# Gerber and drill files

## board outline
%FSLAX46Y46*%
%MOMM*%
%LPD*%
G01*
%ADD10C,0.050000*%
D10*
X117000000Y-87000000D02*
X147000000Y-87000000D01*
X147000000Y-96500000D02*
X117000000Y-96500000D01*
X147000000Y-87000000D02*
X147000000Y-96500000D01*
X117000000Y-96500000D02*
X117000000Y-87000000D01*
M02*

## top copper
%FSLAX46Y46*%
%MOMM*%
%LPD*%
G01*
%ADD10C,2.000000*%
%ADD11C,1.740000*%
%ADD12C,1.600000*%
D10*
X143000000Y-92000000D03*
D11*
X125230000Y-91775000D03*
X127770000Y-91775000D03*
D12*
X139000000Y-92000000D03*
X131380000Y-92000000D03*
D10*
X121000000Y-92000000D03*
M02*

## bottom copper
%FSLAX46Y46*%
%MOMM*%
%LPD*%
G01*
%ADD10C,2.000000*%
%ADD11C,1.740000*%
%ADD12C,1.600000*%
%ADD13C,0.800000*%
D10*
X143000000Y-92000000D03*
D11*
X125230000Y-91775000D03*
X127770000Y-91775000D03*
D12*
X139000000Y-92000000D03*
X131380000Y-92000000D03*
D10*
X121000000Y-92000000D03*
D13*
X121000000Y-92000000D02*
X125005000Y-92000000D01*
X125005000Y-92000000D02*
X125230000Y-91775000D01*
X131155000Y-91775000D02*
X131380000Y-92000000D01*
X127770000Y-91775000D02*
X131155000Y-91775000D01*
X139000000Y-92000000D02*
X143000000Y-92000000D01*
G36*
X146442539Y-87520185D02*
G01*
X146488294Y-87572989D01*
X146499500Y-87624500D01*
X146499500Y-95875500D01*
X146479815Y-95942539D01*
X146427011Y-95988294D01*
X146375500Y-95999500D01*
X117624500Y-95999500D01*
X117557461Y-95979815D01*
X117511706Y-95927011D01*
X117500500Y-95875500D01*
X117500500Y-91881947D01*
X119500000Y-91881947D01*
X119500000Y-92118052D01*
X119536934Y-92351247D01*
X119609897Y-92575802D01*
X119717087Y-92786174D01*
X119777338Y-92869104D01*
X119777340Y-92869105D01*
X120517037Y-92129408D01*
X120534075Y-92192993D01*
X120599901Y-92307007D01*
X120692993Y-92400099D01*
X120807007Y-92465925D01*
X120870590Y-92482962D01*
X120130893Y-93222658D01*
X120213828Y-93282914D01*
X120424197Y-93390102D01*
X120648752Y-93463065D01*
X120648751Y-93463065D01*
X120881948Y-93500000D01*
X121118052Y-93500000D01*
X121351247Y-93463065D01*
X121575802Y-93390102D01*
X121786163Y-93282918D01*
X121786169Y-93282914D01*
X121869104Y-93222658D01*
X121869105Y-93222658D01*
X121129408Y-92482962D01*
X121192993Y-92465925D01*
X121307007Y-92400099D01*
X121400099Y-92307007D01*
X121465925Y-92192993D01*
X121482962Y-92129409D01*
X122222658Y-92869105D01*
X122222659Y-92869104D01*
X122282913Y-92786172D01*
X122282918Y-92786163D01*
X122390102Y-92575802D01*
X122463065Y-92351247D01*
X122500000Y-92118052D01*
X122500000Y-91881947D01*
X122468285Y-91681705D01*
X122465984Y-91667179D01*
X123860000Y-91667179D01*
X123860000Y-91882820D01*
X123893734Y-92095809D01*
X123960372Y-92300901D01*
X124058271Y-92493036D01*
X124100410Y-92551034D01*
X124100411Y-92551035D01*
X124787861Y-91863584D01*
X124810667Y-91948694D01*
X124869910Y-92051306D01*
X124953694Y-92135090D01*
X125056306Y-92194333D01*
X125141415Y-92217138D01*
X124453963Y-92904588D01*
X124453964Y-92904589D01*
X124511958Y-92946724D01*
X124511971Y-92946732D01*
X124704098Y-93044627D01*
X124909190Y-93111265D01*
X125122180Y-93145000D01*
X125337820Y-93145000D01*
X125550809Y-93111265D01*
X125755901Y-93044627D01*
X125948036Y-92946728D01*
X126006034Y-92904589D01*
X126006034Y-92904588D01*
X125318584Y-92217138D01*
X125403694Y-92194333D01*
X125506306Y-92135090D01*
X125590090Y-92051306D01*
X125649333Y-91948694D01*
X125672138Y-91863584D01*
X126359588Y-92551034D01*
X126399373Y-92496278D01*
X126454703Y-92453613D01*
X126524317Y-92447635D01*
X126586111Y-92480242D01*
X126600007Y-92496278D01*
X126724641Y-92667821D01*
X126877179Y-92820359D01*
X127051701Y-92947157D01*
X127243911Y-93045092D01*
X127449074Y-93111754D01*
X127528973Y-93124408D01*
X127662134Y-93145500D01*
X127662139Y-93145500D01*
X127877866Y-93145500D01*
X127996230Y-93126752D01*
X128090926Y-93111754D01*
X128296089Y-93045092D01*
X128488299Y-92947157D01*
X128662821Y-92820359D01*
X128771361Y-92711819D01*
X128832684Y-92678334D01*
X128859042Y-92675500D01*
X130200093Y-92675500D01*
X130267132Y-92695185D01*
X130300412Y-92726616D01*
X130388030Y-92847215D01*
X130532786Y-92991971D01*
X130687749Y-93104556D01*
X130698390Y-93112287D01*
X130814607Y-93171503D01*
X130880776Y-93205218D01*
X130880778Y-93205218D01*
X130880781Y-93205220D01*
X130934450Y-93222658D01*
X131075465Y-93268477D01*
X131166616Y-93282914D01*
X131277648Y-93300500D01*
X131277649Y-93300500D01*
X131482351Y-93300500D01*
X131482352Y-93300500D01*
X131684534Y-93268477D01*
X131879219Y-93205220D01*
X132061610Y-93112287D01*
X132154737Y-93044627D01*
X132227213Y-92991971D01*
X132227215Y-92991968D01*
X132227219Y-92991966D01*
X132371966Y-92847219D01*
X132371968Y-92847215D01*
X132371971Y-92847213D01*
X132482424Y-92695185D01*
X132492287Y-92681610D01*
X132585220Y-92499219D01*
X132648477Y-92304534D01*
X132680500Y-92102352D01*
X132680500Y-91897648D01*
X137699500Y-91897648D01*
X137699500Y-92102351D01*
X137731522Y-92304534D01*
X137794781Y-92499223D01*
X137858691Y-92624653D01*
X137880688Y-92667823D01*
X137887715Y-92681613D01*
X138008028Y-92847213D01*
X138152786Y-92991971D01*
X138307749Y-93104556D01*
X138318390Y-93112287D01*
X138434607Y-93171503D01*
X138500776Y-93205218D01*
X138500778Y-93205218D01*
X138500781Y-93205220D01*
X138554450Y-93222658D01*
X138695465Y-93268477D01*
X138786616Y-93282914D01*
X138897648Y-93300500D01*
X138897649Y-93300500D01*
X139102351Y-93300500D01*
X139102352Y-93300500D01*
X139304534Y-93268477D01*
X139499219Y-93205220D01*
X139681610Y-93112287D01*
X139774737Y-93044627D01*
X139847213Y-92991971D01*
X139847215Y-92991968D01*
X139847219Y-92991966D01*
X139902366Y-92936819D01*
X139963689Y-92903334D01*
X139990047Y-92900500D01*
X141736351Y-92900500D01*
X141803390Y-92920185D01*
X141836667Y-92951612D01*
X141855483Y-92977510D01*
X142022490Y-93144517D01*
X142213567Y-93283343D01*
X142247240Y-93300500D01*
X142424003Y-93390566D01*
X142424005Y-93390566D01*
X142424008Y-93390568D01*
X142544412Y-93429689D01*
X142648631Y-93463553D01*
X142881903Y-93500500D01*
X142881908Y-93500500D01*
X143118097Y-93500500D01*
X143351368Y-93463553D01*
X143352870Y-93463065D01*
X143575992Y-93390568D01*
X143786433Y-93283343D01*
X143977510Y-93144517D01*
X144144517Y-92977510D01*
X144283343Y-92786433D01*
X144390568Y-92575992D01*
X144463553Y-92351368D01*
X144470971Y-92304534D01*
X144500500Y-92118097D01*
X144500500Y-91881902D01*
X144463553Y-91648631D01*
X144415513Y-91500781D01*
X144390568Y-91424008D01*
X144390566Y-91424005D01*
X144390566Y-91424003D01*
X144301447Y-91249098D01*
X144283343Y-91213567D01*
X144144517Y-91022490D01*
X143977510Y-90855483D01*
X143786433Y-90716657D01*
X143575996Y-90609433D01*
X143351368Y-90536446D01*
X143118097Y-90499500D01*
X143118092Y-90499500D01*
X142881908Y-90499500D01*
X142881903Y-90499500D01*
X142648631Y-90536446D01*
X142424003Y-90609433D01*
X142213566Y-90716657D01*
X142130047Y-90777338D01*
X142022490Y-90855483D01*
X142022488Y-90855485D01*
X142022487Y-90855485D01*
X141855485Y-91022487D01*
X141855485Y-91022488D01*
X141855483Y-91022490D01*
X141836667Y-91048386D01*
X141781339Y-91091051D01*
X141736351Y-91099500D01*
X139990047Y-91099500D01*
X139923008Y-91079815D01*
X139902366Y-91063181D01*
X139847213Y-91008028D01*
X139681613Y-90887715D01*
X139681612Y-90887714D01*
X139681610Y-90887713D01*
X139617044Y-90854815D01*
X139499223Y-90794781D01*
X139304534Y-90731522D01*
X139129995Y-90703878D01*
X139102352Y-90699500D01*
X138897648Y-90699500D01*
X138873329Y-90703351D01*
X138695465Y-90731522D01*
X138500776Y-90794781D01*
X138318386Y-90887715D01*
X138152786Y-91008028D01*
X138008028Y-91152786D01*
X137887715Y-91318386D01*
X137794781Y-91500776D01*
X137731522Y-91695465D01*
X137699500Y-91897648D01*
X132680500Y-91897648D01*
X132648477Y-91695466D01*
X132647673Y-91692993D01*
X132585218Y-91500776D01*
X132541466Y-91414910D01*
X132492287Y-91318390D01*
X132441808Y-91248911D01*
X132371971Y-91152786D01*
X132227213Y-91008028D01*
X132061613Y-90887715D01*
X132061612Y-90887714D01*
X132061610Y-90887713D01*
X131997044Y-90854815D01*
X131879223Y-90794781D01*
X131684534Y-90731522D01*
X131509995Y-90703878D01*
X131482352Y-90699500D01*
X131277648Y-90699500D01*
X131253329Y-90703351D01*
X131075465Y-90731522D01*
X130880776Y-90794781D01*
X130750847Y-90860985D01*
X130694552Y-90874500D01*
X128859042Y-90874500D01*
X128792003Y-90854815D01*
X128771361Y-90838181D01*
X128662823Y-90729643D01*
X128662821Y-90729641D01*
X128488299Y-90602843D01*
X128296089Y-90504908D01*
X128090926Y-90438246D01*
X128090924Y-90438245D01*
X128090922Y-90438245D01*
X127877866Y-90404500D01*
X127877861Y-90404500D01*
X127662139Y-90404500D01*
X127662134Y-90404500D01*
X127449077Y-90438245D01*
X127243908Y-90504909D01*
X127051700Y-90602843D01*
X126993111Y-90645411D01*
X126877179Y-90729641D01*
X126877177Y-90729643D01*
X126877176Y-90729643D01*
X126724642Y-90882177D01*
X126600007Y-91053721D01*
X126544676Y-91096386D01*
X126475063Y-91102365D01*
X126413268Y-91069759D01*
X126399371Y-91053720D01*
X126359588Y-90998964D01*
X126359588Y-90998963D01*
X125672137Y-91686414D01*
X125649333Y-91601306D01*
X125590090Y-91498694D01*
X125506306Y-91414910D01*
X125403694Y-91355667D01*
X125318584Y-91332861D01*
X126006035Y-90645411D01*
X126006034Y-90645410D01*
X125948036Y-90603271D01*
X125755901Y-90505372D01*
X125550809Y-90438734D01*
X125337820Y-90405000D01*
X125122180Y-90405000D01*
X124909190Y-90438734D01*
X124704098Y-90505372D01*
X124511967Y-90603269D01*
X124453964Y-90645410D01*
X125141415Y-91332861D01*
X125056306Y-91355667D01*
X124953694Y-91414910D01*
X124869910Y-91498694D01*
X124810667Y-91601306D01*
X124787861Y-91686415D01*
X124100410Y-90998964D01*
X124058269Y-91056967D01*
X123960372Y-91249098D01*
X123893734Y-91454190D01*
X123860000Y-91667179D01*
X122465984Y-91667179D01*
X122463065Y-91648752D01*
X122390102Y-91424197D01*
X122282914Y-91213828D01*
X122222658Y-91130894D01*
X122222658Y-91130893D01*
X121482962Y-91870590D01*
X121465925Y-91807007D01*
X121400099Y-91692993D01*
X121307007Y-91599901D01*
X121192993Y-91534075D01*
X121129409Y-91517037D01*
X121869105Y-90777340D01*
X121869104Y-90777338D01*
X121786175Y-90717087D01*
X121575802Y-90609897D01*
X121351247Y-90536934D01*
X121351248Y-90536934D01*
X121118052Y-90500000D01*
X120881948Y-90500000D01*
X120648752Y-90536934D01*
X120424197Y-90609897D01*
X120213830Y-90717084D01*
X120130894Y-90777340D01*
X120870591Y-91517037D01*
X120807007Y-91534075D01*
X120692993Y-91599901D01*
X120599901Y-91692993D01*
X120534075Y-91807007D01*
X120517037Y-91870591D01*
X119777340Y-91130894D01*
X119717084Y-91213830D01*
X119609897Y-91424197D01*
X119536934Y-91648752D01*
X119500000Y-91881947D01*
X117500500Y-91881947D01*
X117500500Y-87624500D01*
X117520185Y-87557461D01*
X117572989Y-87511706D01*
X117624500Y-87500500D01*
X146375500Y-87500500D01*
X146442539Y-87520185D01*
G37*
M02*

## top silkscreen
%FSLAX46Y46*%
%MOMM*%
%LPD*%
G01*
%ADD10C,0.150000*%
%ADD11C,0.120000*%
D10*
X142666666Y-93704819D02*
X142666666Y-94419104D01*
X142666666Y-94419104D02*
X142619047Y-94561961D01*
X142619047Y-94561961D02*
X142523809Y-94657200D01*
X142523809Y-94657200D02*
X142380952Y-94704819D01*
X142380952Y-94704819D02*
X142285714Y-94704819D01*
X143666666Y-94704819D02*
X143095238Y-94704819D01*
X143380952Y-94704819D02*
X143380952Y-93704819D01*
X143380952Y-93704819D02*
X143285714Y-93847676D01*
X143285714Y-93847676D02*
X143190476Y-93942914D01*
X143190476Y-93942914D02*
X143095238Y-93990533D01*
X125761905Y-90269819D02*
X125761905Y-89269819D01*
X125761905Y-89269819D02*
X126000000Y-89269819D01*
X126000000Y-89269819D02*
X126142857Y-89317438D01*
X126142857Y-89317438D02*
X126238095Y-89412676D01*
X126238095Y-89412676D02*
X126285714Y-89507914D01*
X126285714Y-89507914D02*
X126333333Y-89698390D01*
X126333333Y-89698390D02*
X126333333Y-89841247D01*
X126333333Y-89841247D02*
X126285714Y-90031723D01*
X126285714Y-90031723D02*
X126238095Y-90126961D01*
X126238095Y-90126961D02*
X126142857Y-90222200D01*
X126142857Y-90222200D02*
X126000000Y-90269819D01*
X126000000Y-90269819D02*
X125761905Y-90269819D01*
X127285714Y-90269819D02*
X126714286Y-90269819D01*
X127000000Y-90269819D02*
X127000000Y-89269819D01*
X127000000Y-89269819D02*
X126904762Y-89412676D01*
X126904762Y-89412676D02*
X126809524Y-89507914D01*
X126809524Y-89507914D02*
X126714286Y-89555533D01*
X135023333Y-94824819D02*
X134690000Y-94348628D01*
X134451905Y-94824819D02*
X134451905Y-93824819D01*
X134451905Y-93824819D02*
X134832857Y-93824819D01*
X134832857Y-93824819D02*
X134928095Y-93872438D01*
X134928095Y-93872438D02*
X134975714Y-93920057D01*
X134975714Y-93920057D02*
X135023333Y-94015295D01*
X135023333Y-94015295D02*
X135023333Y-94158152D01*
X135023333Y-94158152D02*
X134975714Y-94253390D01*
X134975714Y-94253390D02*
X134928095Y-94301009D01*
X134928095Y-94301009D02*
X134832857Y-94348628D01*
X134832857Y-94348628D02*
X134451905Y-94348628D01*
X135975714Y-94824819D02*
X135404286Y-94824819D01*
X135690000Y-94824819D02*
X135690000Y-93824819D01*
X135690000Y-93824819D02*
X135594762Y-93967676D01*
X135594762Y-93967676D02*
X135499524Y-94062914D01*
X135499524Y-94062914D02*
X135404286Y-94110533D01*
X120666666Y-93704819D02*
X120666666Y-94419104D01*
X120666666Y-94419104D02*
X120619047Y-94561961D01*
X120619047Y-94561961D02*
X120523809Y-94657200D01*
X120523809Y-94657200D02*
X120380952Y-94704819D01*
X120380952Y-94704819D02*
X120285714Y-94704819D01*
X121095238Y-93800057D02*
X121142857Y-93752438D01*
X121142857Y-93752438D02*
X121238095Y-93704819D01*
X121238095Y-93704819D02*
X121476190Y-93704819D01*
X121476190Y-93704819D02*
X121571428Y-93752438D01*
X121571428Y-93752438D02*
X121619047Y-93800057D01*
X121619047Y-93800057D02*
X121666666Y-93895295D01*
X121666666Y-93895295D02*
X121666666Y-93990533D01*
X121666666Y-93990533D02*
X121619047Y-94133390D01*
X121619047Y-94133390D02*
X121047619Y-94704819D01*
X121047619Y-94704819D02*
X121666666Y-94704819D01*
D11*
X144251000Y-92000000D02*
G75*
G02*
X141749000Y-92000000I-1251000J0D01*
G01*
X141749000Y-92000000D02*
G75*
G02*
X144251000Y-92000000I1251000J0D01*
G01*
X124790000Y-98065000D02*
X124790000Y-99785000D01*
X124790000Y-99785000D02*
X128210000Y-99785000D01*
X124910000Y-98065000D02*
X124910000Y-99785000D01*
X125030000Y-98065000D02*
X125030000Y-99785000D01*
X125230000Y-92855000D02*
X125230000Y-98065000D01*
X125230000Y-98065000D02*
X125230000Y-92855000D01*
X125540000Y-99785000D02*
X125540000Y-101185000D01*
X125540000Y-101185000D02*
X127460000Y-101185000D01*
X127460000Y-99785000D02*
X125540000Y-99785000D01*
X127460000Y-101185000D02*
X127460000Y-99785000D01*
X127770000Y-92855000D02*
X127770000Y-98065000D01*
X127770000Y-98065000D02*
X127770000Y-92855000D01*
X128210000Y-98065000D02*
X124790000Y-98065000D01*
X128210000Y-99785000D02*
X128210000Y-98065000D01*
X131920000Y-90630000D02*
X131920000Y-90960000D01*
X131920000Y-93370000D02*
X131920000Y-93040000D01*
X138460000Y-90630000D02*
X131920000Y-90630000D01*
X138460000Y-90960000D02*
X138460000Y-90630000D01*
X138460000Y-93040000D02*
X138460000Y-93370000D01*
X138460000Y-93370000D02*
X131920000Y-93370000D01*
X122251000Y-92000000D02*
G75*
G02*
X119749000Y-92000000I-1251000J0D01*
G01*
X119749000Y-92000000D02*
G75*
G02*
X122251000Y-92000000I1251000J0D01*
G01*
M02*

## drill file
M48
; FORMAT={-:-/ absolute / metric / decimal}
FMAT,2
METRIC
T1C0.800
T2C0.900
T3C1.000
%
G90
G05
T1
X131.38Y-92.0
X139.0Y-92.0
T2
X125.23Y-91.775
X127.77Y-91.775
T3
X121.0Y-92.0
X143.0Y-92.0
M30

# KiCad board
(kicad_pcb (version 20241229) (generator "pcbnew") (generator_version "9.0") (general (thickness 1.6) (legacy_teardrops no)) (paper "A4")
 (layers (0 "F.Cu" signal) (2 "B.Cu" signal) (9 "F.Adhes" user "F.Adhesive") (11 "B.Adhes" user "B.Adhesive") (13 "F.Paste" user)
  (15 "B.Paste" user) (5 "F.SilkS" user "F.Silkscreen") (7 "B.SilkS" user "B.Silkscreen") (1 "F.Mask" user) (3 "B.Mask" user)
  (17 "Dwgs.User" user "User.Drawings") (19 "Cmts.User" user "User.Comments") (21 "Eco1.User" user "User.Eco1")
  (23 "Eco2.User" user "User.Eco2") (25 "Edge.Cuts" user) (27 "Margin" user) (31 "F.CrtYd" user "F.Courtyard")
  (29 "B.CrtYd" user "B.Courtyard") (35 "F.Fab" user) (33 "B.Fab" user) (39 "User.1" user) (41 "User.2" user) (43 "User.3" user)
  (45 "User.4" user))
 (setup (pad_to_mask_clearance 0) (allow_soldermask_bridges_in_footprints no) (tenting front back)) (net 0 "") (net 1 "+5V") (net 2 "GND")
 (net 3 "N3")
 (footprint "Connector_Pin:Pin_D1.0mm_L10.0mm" (layer "F.Cu") (at 143 92)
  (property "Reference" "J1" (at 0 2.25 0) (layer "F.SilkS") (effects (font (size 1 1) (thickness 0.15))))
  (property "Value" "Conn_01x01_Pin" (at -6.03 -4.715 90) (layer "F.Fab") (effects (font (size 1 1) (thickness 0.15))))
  (fp_circle (center 0 0) (end 1.25 0.05) (stroke (width 0.12) (type solid)) (fill no) (layer "F.SilkS"))
  (pad "1" thru_hole circle (at 0 0) (size 2 2) (drill 1) (layers "*.Cu" "*.Mask") (remove_unused_layers no) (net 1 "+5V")))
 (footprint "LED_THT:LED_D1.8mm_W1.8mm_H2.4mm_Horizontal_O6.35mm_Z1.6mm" (layer "F.Cu") (at 125.23 91.775)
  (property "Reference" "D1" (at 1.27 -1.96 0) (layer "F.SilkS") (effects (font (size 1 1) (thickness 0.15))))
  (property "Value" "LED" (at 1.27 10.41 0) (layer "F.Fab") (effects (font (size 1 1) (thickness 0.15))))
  (fp_line (start -0.44 6.29) (end -0.44 8.01) (stroke (width 0.12) (type solid)) (layer "F.SilkS"))
  (fp_line (start -0.44 8.01) (end 2.98 8.01) (stroke (width 0.12) (type solid)) (layer "F.SilkS"))
  (fp_line (start -0.32 6.29) (end -0.32 8.01) (stroke (width 0.12) (type solid)) (layer "F.SilkS"))
  (fp_line (start -0.2 6.29) (end -0.2 8.01) (stroke (width 0.12) (type solid)) (layer "F.SilkS"))
  (fp_line (start 0 1.08) (end 0 6.29) (stroke (width 0.12) (type solid)) (layer "F.SilkS"))
  (fp_line (start 0 6.29) (end 0 1.08) (stroke (width 0.12) (type solid)) (layer "F.SilkS"))
  (fp_line (start 0.31 8.01) (end 0.31 9.41) (stroke (width 0.12) (type solid)) (layer "F.SilkS"))
  (fp_line (start 0.31 9.41) (end 2.23 9.41) (stroke (width 0.12) (type solid)) (layer "F.SilkS"))
  (fp_line (start 2.23 8.01) (end 0.31 8.01) (stroke (width 0.12) (type solid)) (layer "F.SilkS"))
  (fp_line (start 2.23 9.41) (end 2.23 8.01) (stroke (width 0.12) (type solid)) (layer "F.SilkS"))
  (fp_line (start 2.54 1.08) (end 2.54 6.29) (stroke (width 0.12) (type solid)) (layer "F.SilkS"))
  (fp_line (start 2.54 6.29) (end 2.54 1.08) (stroke (width 0.12) (type solid)) (layer "F.SilkS"))
  (fp_line (start 2.98 6.29) (end -0.44 6.29) (stroke (width 0.12) (type solid)) (layer "F.SilkS"))
  (fp_line (start 2.98 8.01) (end 2.98 6.29) (stroke (width 0.12) (type solid)) (layer "F.SilkS"))
  (pad "1" thru_hole circle (at 0 0) (size 1.74 1.74) (drill 0.9) (layers "*.Cu" "*.Mask") (remove_unused_layers no) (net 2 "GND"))
  (pad "2" thru_hole circle (at 2.54 0) (size 1.74 1.74) (drill 0.9) (layers "*.Cu" "*.Mask") (remove_unused_layers no) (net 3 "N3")))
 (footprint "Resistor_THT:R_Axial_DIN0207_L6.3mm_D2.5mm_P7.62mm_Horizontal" (layer "F.Cu") (at 139 92 180)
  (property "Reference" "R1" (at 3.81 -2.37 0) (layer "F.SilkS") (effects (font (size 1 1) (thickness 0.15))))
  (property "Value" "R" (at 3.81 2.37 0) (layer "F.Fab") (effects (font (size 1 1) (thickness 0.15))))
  (fp_line (start 7.08 1.37) (end 7.08 1.04) (stroke (width 0.12) (type solid)) (layer "F.SilkS"))
  (fp_line (start 7.08 -1.37) (end 7.08 -1.04) (stroke (width 0.12) (type solid)) (layer "F.SilkS"))
  (fp_line (start 0.54 1.37) (end 7.08 1.37) (stroke (width 0.12) (type solid)) (layer "F.SilkS"))
  (fp_line (start 0.54 1.04) (end 0.54 1.37) (stroke (width 0.12) (type solid)) (layer "F.SilkS"))
  (fp_line (start 0.54 -1.04) (end 0.54 -1.37) (stroke (width 0.12) (type solid)) (layer "F.SilkS"))
  (fp_line (start 0.54 -1.37) (end 7.08 -1.37) (stroke (width 0.12) (type solid)) (layer "F.SilkS"))
  (pad "1" thru_hole circle (at 0 0 180) (size 1.6 1.6) (drill 0.8) (layers "*.Cu" "*.Mask") (remove_unused_layers no) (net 1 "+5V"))
  (pad "2" thru_hole circle (at 7.62 0 180) (size 1.6 1.6) (drill 0.8) (layers "*.Cu" "*.Mask") (remove_unused_layers no) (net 3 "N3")))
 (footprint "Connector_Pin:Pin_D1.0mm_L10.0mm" (layer "F.Cu") (at 121 92)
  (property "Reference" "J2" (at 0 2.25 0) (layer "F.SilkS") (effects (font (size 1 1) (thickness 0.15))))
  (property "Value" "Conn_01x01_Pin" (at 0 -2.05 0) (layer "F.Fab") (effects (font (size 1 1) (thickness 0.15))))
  (fp_circle (center 0 0) (end 1.25 0.05) (stroke (width 0.12) (type solid)) (fill no) (layer "F.SilkS"))
  (pad "1" thru_hole circle (at 0 0) (size 2 2) (drill 1) (layers "*.Cu" "*.Mask") (remove_unused_layers no) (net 2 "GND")))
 (gr_line (start 117 87) (end 147 87) (stroke (width 0.05) (type default)) (layer "Edge.Cuts"))
 (gr_line (start 147 96.5) (end 117 96.5) (stroke (width 0.05) (type default)) (layer "Edge.Cuts"))
 (gr_line (start 147 87) (end 147 96.5) (stroke (width 0.05) (type default)) (layer "Edge.Cuts"))
 (gr_line (start 117 96.5) (end 117 87) (stroke (width 0.05) (type default)) (layer "Edge.Cuts"))
 (segment (start 121 92) (end 125.005 92) (width 0.8) (layer "B.Cu") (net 2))
 (segment (start 125.005 92) (end 125.23 91.775) (width 0.8) (layer "B.Cu") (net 2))
 (segment (start 131.155 91.775) (end 131.38 92) (width 0.8) (layer "B.Cu") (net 3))
 (segment (start 127.77 91.775) (end 131.155 91.775) (width 0.8) (layer "B.Cu") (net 3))
 (segment (start 139 92) (end 143 92) (width 0.8) (layer "B.Cu") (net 1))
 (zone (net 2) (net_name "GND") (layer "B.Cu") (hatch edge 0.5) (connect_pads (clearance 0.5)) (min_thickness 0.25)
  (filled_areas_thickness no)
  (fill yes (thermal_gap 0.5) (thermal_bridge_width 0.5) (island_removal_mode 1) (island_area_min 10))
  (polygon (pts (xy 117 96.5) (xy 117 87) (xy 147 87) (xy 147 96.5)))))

